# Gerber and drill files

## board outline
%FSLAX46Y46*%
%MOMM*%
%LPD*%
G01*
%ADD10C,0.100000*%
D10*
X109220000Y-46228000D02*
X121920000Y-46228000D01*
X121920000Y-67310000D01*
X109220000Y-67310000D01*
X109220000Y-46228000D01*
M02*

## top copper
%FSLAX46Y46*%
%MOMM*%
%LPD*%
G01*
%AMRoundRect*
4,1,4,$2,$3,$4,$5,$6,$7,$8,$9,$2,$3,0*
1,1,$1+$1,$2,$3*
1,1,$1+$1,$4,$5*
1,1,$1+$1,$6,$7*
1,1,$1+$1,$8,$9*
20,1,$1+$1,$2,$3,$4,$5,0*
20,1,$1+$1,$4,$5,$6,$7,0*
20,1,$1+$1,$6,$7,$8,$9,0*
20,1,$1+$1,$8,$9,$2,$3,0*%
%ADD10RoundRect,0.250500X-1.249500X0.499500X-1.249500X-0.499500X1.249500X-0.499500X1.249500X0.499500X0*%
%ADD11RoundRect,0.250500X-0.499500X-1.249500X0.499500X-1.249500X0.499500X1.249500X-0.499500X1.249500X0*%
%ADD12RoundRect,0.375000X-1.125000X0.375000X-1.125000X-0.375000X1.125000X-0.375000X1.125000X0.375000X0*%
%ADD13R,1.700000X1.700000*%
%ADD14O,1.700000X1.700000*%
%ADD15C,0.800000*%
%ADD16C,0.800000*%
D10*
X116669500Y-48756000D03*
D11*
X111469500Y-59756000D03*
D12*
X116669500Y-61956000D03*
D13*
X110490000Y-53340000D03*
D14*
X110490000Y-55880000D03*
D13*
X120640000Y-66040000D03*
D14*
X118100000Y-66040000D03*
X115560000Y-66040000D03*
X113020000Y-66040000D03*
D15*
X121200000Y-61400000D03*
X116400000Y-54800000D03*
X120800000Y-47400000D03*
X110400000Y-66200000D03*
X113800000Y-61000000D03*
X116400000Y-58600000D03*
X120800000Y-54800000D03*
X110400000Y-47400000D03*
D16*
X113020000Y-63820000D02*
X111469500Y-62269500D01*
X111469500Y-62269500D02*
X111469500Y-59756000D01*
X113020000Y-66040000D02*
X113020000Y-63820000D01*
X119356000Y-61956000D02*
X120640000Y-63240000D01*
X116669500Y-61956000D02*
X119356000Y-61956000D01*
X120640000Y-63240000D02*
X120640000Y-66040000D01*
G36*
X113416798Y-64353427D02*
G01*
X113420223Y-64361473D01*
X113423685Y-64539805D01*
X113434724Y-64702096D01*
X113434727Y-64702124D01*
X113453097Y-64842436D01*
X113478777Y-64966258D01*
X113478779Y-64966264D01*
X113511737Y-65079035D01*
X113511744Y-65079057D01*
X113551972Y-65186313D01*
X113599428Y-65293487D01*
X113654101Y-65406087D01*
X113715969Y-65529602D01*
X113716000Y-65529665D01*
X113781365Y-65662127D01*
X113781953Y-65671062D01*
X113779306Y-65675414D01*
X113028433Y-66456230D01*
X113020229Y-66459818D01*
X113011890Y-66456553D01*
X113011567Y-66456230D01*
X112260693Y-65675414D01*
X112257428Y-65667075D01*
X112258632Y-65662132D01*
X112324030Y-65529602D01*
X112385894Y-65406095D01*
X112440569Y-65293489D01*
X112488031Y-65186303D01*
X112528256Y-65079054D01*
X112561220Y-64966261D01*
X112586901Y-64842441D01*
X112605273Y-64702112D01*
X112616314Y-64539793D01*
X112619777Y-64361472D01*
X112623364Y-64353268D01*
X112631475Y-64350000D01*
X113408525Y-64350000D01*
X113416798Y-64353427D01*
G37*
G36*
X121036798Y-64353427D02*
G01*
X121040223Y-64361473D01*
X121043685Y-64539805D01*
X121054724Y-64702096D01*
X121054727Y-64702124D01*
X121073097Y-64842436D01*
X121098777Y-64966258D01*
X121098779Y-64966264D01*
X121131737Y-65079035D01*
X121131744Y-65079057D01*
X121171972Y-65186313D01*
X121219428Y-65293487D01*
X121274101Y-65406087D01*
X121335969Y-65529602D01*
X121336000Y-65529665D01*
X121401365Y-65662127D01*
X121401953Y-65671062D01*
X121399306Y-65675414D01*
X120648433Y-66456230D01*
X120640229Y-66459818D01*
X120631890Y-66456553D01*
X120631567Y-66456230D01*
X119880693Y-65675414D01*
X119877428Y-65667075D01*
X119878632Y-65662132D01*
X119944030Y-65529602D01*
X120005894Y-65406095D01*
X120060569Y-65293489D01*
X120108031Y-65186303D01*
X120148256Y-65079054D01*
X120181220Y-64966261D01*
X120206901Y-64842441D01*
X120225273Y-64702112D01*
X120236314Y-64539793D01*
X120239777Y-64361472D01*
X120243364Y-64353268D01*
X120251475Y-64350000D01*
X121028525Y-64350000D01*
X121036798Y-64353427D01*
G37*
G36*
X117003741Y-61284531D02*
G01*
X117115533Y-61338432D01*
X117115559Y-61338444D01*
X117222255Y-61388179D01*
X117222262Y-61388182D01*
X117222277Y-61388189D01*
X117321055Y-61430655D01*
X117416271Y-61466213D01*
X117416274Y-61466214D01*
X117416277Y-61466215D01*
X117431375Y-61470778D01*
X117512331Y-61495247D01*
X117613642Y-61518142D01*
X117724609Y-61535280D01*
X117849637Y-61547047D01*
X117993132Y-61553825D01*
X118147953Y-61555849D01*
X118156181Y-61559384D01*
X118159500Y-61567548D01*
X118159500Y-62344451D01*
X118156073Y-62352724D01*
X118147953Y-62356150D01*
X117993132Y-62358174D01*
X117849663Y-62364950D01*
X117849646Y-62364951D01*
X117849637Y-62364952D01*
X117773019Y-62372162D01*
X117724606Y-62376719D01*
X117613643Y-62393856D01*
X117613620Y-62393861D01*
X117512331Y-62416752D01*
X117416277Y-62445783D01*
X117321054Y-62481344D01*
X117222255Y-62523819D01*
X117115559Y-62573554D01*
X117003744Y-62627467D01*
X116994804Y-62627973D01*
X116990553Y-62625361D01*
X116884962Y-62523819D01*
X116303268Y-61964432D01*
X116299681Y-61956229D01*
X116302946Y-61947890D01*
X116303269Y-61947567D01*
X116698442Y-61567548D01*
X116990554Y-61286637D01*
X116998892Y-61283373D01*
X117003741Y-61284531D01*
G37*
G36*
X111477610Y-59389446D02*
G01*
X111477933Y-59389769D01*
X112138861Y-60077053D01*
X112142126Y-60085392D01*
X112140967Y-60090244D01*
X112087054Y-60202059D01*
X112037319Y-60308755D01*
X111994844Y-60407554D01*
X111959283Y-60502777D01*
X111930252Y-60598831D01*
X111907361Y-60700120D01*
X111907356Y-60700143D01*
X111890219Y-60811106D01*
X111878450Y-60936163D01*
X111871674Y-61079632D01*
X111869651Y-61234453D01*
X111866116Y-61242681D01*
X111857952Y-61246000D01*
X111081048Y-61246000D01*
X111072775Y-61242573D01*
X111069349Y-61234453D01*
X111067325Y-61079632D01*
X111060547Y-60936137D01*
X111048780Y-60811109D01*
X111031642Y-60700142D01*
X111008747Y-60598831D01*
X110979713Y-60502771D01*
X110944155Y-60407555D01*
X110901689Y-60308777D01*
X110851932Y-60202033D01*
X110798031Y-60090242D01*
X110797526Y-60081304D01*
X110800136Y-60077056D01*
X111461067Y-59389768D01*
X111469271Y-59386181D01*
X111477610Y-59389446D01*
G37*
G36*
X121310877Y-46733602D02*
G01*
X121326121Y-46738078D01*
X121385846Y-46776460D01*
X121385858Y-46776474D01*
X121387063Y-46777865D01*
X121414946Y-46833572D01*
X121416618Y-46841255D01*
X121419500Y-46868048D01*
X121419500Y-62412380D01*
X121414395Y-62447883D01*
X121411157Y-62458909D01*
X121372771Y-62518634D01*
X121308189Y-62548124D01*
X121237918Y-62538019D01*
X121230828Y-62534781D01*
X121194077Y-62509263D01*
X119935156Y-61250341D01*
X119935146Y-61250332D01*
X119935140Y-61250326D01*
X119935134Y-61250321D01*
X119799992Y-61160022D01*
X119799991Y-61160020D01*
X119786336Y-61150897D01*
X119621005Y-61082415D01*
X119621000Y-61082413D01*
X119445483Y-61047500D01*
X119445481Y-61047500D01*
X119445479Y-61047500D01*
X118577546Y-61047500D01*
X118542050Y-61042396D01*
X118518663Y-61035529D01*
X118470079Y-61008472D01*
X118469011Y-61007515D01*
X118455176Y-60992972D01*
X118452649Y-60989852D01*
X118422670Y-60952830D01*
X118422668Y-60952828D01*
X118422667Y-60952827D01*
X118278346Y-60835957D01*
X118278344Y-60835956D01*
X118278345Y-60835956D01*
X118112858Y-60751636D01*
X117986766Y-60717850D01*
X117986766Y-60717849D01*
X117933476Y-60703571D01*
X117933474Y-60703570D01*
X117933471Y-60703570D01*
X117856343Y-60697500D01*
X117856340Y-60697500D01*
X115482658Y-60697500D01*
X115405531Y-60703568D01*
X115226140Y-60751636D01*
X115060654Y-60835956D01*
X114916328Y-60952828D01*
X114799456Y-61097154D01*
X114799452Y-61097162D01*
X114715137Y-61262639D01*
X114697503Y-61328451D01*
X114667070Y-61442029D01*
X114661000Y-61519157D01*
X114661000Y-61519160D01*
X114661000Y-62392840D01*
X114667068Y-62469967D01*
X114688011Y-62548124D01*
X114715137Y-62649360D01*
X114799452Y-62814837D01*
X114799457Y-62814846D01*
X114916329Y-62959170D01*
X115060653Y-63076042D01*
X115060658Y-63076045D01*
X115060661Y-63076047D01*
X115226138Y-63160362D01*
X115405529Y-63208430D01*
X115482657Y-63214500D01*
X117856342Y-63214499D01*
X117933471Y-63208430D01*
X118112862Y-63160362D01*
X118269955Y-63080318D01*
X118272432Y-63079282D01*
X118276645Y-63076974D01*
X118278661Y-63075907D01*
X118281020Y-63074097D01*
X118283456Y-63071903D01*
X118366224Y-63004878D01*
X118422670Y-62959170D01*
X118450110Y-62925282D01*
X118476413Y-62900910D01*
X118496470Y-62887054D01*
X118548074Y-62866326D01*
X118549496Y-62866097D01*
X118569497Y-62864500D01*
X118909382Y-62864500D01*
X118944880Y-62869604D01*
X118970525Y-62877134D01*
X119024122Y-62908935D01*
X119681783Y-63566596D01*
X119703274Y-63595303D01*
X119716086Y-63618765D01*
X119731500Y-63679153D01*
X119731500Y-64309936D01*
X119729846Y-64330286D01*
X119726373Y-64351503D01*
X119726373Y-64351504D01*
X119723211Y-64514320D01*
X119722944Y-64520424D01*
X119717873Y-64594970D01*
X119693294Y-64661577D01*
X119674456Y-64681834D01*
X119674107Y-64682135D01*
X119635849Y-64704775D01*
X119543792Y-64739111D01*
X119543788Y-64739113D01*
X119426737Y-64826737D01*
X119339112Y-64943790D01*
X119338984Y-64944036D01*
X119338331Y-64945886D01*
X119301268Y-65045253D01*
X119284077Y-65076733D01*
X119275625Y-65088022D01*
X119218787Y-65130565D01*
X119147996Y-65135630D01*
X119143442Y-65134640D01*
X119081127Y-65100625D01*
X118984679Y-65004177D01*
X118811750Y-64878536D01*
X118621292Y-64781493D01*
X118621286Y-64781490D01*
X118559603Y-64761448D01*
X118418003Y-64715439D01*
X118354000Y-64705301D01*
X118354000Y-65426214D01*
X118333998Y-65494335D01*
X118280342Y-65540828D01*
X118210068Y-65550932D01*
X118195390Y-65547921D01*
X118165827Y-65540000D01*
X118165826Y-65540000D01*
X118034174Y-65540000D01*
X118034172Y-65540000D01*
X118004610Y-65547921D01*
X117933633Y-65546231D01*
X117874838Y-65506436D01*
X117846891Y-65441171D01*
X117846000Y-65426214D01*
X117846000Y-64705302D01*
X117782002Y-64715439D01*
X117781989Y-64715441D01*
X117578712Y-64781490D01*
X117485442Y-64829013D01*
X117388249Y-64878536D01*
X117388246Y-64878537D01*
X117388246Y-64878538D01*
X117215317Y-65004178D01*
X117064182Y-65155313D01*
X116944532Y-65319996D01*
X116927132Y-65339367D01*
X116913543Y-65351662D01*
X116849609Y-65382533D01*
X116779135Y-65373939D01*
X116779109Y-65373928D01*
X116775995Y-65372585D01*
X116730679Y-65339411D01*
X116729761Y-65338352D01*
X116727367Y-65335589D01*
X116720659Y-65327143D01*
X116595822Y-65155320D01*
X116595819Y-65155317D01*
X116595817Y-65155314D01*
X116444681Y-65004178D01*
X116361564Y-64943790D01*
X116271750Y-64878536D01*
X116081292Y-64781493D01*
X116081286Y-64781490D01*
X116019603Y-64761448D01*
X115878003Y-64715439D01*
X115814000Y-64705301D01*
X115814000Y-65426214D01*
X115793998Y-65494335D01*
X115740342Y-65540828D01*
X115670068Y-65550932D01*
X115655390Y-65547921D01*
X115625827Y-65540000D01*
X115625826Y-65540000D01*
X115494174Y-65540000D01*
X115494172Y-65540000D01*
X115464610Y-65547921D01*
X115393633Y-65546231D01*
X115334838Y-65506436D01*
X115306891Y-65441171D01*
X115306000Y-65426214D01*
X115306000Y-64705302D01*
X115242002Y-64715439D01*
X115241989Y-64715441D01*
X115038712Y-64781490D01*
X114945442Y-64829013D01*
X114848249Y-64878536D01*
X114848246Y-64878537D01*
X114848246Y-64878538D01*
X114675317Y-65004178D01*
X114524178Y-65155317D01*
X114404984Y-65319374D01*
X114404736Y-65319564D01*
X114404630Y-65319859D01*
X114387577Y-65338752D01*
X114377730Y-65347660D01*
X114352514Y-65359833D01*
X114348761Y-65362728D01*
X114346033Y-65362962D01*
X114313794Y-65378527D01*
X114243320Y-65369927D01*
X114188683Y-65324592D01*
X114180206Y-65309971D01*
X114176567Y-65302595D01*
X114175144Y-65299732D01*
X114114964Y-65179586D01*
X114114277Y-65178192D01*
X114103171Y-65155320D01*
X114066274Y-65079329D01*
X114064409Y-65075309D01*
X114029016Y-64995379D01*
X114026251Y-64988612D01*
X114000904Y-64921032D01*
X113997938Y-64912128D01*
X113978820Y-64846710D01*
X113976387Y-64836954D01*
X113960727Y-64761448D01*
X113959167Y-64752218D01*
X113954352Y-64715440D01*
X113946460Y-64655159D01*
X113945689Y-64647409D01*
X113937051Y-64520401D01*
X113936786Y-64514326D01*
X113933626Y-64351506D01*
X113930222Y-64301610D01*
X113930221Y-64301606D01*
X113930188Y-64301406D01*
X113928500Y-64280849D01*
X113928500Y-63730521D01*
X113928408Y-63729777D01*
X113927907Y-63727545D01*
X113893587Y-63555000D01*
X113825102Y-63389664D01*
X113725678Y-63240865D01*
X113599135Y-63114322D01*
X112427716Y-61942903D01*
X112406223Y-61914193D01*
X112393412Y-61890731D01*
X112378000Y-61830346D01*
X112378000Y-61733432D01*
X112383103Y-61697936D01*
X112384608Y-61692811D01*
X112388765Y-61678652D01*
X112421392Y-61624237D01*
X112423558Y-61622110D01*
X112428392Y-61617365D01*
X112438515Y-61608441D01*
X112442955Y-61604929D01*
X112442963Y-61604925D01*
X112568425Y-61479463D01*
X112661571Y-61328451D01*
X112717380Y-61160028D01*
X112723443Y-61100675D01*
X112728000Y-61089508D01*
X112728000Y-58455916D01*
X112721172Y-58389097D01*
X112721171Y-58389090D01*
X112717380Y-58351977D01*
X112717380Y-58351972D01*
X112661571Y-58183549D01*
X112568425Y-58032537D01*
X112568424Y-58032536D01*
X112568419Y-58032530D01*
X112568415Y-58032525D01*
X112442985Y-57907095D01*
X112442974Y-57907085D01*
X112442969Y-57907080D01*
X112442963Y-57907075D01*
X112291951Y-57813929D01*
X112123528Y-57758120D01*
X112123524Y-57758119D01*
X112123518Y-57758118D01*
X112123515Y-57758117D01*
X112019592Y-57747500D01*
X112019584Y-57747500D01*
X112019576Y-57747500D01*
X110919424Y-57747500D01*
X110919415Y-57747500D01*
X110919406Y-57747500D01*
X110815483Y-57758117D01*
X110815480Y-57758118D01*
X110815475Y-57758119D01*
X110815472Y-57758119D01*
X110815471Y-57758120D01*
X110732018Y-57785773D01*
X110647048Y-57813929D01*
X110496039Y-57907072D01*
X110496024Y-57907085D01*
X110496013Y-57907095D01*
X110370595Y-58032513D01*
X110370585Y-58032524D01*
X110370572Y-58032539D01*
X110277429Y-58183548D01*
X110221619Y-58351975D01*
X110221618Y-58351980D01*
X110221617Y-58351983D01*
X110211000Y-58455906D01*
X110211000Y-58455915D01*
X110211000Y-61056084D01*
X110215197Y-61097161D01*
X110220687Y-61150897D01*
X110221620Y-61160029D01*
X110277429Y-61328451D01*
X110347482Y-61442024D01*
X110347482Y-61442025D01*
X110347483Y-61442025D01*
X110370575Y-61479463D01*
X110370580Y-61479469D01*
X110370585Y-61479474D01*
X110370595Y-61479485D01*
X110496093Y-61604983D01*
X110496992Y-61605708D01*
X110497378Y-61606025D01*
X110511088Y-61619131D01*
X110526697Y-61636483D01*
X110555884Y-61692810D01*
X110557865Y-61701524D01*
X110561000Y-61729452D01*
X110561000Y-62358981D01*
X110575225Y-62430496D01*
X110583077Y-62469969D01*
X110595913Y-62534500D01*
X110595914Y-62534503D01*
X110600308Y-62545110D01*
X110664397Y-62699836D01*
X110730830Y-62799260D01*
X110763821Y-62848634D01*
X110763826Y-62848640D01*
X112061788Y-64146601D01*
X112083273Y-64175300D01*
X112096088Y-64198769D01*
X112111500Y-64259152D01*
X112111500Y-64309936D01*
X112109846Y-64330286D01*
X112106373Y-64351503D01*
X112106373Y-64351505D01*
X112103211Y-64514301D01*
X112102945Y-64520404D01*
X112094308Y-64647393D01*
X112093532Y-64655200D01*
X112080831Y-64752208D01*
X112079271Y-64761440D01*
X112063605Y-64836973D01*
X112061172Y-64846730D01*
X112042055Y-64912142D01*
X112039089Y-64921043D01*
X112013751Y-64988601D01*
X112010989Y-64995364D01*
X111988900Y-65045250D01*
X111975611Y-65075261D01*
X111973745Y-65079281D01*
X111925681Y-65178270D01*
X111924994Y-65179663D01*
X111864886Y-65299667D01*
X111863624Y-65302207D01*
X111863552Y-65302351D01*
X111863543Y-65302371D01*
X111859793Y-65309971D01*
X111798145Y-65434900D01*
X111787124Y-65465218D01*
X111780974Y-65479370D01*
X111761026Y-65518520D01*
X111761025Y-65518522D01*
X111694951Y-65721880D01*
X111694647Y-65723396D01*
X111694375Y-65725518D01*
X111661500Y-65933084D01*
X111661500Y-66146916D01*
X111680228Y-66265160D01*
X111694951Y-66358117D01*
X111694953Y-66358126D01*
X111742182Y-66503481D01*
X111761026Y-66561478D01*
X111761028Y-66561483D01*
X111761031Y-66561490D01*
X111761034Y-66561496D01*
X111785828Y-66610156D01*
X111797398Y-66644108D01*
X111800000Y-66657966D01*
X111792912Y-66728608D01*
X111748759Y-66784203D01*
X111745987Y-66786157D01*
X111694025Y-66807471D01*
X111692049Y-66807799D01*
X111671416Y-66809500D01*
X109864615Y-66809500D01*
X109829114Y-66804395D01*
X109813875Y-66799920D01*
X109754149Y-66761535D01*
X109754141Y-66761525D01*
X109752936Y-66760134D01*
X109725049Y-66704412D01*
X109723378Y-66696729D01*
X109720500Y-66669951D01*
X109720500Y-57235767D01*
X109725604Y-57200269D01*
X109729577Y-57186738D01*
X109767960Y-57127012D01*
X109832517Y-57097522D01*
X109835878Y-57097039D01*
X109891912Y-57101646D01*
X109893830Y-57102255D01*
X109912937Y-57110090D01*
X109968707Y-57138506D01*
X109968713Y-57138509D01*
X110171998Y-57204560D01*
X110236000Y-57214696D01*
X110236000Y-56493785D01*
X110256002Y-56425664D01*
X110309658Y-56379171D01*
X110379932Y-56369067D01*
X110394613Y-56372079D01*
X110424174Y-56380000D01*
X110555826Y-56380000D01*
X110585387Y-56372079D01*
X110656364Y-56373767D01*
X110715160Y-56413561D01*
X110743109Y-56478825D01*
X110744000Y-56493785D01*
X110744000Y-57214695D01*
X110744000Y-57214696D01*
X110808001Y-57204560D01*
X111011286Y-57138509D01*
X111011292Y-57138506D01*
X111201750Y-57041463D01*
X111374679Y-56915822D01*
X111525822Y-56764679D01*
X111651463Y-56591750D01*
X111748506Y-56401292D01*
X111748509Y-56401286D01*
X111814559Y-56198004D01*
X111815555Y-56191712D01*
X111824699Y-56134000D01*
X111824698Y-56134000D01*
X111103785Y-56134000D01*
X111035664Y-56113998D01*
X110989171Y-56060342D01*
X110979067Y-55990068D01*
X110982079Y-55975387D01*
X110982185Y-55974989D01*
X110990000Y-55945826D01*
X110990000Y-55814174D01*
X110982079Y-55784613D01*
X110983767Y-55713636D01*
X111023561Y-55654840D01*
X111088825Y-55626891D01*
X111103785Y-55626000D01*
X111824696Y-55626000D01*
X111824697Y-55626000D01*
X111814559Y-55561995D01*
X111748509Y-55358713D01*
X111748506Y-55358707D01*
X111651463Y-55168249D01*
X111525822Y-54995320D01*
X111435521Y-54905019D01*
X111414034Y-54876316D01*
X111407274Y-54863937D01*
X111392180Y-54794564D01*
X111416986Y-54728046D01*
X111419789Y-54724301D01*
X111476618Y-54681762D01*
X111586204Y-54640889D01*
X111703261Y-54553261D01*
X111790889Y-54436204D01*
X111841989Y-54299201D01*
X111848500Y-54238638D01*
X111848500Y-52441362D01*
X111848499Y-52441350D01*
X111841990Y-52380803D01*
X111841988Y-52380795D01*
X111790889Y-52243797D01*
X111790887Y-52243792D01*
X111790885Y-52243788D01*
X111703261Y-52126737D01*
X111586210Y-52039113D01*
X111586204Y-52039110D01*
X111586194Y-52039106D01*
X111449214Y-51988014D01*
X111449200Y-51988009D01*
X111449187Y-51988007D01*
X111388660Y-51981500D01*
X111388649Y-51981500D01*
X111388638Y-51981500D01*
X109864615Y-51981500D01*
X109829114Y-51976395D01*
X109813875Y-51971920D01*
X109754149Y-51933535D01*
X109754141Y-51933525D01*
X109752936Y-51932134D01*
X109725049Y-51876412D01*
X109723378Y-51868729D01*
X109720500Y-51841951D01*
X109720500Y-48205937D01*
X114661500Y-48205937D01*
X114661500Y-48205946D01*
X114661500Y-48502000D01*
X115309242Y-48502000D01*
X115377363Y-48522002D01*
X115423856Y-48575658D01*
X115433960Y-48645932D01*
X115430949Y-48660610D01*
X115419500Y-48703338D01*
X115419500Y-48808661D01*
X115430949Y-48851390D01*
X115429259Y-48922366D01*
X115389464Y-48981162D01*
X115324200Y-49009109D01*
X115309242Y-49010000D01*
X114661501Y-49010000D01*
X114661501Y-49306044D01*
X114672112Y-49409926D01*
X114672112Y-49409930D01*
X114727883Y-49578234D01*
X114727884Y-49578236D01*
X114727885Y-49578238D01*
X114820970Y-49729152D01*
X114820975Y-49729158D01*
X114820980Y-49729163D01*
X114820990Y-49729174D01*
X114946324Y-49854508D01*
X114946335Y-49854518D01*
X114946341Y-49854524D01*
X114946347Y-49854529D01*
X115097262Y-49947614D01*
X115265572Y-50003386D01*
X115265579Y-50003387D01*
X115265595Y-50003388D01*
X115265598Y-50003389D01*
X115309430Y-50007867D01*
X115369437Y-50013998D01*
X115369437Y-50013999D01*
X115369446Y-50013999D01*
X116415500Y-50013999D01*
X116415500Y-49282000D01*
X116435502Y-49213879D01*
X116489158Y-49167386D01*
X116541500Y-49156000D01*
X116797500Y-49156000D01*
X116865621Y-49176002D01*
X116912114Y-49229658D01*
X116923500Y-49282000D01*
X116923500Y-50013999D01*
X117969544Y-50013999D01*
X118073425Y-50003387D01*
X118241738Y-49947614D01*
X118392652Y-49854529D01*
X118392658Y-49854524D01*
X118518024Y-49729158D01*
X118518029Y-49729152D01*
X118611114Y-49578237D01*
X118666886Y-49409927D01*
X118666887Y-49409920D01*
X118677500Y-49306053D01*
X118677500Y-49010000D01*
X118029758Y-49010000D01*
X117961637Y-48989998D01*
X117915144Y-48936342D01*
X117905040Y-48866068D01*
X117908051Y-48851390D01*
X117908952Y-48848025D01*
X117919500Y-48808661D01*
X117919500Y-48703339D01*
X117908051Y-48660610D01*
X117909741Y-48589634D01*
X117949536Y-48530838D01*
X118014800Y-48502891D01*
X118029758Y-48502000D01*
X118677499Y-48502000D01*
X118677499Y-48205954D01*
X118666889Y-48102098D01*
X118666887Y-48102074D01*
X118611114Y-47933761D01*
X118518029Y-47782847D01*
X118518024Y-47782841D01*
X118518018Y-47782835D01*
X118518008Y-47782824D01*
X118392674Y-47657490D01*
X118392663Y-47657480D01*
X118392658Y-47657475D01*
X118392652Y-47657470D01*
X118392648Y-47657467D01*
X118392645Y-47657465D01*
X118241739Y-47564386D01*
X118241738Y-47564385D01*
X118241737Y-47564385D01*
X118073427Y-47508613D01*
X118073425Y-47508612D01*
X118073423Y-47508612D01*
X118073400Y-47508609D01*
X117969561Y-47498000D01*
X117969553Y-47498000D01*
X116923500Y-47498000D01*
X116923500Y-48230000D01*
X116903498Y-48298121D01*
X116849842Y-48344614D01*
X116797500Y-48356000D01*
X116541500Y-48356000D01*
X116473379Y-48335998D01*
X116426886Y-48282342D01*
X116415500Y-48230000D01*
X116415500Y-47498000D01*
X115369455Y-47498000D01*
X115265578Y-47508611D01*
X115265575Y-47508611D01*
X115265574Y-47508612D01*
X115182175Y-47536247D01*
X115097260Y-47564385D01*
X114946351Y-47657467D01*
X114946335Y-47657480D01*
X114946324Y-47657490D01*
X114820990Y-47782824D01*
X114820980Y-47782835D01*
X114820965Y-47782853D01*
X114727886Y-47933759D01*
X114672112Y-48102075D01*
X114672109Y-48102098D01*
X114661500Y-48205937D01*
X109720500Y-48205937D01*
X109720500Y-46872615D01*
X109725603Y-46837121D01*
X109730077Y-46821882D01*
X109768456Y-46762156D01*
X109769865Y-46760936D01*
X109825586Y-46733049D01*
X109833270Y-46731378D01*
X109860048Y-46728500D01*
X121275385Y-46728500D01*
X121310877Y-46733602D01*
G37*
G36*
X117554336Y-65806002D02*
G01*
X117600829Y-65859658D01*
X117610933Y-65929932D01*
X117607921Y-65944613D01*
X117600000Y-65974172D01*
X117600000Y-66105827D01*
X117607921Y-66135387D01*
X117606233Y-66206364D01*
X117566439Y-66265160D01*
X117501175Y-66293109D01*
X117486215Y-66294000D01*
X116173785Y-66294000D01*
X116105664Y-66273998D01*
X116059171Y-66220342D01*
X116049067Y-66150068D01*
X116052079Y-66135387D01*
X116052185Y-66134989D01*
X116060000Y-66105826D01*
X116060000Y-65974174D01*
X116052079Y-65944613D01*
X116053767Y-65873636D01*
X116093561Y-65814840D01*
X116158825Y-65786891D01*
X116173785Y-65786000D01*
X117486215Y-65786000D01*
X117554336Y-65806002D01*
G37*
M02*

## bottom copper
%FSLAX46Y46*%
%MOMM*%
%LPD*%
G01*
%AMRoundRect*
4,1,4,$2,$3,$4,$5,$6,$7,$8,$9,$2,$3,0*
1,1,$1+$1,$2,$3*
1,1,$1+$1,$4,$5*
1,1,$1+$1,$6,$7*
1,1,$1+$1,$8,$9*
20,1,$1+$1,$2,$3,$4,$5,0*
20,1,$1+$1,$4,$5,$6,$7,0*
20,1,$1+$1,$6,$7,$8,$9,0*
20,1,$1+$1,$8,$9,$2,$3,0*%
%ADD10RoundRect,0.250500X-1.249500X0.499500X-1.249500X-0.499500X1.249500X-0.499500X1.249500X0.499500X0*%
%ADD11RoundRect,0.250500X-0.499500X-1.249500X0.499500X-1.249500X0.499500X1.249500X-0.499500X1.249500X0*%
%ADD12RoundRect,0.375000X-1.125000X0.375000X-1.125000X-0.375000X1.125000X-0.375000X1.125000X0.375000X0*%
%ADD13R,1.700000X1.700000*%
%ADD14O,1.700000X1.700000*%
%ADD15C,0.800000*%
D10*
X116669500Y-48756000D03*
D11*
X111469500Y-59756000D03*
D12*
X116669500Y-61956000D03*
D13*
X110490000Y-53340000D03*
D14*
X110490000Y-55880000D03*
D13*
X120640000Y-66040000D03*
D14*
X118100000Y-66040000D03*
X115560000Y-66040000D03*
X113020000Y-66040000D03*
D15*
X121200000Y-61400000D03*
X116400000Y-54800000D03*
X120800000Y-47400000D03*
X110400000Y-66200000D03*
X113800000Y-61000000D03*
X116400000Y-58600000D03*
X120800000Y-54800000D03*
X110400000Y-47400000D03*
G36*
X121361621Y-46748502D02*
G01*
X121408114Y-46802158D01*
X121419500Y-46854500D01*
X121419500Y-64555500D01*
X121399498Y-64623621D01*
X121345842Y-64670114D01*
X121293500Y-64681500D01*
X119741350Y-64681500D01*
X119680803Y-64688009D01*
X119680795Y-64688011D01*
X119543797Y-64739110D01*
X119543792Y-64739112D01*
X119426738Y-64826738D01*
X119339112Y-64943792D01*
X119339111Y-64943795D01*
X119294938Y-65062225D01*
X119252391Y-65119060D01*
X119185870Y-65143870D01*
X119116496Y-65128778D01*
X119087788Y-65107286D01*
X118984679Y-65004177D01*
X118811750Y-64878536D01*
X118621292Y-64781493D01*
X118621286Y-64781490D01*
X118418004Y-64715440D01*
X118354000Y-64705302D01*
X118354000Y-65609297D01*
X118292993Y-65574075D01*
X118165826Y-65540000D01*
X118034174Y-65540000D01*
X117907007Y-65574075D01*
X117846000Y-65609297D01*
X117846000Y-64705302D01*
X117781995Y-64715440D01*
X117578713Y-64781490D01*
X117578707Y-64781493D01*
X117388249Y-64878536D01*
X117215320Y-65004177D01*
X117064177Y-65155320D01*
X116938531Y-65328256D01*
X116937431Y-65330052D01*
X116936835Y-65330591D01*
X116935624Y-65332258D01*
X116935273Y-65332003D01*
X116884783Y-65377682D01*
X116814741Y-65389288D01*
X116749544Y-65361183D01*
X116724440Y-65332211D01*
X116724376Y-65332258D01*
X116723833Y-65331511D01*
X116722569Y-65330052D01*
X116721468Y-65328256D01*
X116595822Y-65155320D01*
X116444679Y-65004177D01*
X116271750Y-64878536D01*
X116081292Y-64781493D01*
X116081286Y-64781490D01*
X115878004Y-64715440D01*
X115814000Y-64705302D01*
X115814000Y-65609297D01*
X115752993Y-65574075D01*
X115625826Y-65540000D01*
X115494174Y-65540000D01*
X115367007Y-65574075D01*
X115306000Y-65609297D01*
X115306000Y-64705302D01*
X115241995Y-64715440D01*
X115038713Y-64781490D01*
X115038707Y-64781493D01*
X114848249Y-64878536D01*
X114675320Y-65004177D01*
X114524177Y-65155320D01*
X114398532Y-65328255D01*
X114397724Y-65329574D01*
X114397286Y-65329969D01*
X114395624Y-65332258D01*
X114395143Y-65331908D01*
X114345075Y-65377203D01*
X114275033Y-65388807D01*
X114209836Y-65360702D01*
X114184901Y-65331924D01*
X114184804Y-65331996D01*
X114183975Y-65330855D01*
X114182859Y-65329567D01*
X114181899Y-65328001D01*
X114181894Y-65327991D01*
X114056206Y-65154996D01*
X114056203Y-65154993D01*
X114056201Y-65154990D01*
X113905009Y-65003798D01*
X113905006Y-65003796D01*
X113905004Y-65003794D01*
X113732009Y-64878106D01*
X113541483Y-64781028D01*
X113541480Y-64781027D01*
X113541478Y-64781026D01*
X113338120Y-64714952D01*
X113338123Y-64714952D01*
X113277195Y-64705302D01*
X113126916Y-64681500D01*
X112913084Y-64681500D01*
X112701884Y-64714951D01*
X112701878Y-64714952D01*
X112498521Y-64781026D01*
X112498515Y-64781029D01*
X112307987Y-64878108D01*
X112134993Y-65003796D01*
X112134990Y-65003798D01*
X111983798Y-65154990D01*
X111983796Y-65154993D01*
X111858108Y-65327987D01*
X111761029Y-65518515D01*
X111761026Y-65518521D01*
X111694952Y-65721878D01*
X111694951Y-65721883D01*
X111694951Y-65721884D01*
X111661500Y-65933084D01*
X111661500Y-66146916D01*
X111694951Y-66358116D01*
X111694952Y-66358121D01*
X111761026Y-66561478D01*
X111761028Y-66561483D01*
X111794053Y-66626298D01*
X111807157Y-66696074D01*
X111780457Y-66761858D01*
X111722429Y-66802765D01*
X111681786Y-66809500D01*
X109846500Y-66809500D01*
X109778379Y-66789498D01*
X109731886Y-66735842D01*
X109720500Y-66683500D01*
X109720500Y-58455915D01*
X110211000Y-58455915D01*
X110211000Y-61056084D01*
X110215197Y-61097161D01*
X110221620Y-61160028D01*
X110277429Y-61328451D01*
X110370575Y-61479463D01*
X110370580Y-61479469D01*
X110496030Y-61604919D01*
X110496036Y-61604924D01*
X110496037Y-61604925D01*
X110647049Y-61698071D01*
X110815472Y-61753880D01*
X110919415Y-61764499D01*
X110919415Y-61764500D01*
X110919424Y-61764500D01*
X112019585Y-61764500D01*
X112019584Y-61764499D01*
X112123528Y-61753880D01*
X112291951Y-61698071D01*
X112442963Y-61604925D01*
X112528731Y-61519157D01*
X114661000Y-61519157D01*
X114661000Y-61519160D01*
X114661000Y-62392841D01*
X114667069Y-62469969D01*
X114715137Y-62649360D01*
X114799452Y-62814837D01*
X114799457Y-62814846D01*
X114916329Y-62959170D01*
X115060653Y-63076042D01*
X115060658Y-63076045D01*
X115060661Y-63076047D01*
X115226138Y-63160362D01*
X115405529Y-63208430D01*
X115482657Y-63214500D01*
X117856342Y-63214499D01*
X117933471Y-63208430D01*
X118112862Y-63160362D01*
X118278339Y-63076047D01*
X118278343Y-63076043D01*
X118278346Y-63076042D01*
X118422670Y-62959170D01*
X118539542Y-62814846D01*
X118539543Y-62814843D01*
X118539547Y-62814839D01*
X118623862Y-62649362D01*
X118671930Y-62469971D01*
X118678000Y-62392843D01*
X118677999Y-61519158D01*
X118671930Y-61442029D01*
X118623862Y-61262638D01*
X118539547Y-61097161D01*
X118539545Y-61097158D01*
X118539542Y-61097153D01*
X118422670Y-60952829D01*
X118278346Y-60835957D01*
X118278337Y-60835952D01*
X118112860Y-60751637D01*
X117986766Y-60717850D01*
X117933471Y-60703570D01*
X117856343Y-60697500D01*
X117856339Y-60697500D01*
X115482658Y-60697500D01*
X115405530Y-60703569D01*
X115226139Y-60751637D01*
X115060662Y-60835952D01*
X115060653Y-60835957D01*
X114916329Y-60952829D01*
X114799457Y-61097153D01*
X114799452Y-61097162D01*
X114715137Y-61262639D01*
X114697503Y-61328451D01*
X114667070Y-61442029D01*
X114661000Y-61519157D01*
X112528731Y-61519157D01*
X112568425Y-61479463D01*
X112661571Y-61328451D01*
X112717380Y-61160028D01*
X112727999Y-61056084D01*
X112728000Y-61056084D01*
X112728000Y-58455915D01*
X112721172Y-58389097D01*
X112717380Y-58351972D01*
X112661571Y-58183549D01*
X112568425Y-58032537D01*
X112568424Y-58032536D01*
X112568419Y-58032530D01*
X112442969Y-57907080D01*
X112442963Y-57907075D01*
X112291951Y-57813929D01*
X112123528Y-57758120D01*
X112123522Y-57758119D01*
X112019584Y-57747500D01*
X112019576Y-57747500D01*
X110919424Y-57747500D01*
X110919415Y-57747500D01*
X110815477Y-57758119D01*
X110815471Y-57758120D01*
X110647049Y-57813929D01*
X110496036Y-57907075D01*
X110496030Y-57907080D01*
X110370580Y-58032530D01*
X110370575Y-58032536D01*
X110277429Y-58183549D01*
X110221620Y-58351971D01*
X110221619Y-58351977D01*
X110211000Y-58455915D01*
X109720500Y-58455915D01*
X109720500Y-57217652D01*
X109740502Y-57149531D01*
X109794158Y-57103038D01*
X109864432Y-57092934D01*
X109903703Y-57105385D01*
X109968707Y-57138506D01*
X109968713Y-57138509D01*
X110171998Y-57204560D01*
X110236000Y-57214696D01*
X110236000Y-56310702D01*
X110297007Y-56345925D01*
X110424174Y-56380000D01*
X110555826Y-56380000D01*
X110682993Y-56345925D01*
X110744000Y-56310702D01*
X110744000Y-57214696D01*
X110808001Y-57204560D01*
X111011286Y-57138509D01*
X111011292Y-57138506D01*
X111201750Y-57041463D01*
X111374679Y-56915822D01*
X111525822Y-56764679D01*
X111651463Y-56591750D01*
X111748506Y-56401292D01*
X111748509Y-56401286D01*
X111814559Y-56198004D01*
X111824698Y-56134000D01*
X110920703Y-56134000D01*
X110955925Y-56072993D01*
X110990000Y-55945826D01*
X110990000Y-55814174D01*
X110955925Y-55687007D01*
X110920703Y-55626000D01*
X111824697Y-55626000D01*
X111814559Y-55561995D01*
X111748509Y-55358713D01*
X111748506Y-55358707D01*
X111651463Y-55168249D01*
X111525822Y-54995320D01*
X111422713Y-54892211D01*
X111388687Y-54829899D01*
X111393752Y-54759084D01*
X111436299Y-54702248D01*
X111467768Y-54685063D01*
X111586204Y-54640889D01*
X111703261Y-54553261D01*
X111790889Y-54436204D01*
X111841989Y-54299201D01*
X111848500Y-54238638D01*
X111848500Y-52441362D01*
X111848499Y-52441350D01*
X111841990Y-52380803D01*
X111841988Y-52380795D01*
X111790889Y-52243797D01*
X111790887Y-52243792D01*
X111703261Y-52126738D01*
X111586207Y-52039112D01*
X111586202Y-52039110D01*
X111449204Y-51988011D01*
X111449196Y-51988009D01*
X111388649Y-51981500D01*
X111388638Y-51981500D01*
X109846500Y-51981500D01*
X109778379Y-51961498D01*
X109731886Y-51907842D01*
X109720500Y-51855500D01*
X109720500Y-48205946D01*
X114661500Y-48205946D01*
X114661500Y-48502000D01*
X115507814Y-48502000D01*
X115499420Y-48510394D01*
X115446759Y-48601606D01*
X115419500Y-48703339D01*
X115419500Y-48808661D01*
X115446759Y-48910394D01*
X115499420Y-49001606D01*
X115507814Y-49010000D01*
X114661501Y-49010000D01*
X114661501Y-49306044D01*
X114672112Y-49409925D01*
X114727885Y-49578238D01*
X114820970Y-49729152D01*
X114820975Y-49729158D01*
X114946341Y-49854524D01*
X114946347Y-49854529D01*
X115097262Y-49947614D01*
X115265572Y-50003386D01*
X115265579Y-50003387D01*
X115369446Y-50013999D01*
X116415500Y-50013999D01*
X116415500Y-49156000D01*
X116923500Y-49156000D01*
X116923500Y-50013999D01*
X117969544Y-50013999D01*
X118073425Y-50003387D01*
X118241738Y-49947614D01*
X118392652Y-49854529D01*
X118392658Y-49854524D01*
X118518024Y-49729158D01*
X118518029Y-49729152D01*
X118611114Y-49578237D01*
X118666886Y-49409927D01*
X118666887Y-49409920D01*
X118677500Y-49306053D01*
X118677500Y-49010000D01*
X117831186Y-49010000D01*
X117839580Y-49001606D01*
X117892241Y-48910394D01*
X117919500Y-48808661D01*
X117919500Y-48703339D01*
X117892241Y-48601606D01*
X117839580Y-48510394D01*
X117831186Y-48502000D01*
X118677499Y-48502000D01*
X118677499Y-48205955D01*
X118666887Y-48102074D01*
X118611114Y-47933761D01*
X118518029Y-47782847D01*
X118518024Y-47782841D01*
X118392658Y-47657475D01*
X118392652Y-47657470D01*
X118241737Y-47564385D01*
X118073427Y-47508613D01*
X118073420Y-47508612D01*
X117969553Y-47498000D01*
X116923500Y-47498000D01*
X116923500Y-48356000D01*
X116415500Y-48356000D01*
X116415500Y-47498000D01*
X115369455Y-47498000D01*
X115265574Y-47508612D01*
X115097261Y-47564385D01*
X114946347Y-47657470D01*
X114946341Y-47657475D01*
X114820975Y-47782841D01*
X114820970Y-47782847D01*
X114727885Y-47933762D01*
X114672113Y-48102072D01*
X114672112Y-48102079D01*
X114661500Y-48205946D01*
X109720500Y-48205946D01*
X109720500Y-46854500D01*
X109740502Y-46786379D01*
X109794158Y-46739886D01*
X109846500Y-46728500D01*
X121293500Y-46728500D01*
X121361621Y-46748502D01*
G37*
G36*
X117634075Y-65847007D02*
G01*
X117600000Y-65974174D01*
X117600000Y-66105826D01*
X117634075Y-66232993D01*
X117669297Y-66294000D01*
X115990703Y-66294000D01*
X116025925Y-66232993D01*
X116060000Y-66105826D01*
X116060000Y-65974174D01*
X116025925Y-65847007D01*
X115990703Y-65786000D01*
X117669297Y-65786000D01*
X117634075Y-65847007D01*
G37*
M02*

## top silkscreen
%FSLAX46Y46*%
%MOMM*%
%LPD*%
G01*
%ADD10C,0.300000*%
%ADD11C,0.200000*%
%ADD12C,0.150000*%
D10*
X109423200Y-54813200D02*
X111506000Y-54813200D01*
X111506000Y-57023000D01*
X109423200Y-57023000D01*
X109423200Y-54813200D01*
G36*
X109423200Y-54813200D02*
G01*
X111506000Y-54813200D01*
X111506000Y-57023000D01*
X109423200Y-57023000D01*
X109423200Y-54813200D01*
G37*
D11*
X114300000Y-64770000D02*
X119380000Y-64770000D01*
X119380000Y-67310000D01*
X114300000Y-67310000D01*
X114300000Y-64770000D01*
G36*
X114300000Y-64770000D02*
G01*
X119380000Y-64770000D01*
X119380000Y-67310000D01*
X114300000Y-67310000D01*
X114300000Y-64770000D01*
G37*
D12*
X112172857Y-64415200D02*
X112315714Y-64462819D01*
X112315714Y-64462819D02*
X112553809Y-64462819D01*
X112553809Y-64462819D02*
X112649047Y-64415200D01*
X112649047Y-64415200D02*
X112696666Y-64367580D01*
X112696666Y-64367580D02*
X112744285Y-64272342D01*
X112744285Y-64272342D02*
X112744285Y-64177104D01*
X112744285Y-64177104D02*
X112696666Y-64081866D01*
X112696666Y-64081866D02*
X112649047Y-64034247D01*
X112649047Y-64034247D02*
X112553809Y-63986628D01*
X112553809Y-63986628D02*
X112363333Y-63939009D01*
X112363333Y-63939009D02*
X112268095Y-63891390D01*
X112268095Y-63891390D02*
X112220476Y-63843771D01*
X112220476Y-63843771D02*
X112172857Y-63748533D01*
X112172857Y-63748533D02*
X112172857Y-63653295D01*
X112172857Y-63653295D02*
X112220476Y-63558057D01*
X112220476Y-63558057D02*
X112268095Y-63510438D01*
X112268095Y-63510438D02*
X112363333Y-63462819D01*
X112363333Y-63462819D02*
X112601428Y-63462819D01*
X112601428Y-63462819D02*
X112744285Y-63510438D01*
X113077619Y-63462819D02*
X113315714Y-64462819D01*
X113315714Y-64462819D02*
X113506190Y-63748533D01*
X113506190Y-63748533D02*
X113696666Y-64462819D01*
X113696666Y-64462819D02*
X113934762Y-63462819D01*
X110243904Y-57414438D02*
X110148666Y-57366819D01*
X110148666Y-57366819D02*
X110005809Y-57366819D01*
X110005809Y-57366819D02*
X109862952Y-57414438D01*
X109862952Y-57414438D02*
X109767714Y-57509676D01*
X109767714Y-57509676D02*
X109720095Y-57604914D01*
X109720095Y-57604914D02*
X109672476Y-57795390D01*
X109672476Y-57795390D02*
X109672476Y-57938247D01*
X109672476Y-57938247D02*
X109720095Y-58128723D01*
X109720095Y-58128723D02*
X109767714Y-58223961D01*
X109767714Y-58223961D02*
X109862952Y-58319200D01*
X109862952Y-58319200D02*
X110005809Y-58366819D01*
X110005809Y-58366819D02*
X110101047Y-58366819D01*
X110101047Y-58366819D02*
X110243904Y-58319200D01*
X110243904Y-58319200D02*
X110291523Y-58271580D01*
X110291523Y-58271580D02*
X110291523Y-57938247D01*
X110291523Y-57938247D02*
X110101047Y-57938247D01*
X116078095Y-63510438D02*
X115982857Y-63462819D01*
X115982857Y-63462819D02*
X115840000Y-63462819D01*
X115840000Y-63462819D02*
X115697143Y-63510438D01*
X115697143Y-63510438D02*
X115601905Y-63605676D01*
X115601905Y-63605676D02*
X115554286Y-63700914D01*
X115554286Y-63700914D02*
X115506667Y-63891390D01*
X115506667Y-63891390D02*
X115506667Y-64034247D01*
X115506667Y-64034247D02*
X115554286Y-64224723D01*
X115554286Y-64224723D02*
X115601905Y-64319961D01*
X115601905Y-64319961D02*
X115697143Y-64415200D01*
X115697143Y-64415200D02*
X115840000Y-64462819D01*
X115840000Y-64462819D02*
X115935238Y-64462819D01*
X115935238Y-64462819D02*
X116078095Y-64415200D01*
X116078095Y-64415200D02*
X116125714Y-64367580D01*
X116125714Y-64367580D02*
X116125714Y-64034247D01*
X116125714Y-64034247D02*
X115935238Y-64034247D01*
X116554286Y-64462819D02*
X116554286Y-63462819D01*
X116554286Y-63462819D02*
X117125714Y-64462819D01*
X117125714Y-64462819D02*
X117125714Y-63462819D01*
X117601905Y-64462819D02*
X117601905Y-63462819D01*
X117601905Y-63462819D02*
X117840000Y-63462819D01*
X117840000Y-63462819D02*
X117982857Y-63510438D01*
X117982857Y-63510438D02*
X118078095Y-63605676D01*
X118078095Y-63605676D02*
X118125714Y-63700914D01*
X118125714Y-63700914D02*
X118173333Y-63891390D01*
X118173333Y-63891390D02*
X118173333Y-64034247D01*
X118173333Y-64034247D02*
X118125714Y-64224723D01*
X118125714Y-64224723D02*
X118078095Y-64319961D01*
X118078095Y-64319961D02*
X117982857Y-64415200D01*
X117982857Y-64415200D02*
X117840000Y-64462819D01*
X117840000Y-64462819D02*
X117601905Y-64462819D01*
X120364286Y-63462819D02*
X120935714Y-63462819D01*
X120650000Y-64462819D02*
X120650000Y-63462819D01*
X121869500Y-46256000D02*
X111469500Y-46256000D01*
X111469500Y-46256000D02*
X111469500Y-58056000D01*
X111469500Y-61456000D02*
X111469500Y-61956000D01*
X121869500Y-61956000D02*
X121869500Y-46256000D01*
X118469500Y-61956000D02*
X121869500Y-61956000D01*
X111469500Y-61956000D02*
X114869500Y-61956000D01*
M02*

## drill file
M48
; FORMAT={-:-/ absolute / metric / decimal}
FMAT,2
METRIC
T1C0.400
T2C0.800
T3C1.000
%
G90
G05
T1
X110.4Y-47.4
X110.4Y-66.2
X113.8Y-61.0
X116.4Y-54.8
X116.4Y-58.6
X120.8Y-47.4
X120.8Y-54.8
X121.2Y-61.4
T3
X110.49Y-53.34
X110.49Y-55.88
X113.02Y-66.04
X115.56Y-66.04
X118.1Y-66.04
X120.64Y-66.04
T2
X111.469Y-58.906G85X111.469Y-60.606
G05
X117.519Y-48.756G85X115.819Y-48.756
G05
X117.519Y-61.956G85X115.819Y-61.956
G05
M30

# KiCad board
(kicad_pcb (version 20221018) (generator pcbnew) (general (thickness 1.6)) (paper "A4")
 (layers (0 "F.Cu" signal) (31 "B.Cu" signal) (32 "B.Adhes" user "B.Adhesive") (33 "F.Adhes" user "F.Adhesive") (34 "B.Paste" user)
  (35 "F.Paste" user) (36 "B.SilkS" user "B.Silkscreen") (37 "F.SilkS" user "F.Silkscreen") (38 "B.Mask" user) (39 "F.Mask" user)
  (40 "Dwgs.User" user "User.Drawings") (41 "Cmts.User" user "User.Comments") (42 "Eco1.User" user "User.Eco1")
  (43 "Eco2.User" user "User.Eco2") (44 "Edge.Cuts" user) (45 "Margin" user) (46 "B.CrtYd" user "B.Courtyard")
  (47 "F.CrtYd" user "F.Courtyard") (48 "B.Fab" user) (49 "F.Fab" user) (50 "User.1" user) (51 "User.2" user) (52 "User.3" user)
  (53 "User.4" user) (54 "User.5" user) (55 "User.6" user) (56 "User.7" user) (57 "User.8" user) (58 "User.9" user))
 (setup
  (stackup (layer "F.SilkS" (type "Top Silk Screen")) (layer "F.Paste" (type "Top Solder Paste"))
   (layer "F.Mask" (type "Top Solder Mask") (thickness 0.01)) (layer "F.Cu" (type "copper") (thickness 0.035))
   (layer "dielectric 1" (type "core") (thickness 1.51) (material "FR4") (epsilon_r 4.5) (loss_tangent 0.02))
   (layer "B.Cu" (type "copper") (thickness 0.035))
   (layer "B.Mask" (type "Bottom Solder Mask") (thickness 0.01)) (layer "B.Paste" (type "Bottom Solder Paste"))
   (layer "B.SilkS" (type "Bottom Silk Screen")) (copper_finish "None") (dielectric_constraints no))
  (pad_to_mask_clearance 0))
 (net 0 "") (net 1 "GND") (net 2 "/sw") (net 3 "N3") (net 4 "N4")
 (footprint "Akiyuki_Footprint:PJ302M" (layer "F.Cu") (at 116.6695 46.256 -90)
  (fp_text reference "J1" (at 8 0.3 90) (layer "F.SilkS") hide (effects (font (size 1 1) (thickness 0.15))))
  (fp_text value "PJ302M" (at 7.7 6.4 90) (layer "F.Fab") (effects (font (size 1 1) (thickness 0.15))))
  (fp_line (start 0 -5.2) (end 0 5.2) (stroke (width 0.15) (type solid)) (layer "F.SilkS"))
  (fp_line (start 0 5.2) (end 11.8 5.2) (stroke (width 0.15) (type solid)) (layer "F.SilkS"))
  (fp_line (start 15.2 5.2) (end 15.7 5.2) (stroke (width 0.15) (type solid)) (layer "F.SilkS"))
  (fp_line (start 15.7 -5.2) (end 0 -5.2) (stroke (width 0.15) (type solid)) (layer "F.SilkS"))
  (fp_line (start 15.7 -1.8) (end 15.7 -5.2) (stroke (width 0.15) (type solid)) (layer "F.SilkS"))
  (fp_line (start 15.7 5.2) (end 15.7 1.8) (stroke (width 0.15) (type solid)) (layer "F.SilkS"))
  (pad "1" thru_hole roundrect (at 2.5 0 270) (size 1.5 3) (drill oval 0.8 2.5) (layers "*.Cu" "*.Mask") (roundrect_rratio 0.167)
   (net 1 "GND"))
  (pad "2" thru_hole roundrect (at 13.5 5.2) (size 1.5 3) (drill oval 0.8 2.5) (layers "*.Cu" "*.Mask") (roundrect_rratio 0.167)
   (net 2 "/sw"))
  (pad "3" thru_hole roundrect (at 15.7 0 270) (size 1.5 3) (drill oval 0.8 2.5) (layers "*.Cu" "*.Mask") (roundrect_rratio 0.25)
   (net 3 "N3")))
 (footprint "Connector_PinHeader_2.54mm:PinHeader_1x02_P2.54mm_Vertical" (layer "B.Cu") (at 110.49 53.34 180)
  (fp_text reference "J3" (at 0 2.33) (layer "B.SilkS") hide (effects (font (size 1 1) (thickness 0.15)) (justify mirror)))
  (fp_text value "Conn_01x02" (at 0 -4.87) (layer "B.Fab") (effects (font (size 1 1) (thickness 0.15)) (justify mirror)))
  (pad "1" thru_hole rect (at 0 0 180) (size 1.7 1.7) (drill 1) (layers "*.Cu" "*.Mask") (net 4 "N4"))
  (pad "2" thru_hole oval (at 0 -2.54 180) (size 1.7 1.7) (drill 1) (layers "*.Cu" "*.Mask") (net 1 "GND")))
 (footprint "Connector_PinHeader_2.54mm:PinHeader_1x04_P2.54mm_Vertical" (layer "B.Cu") (at 120.64 66.04 90)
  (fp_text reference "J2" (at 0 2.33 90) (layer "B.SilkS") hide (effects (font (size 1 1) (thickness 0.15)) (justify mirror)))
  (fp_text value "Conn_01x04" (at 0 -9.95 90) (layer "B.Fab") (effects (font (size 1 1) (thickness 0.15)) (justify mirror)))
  (pad "1" thru_hole rect (at 0 0 90) (size 1.7 1.7) (drill 1) (layers "*.Cu" "*.Mask") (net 3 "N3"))
  (pad "2" thru_hole oval (at 0 -2.54 90) (size 1.7 1.7) (drill 1) (layers "*.Cu" "*.Mask") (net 1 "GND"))
  (pad "3" thru_hole oval (at 0 -5.08 90) (size 1.7 1.7) (drill 1) (layers "*.Cu" "*.Mask") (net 1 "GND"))
  (pad "4" thru_hole oval (at 0 -7.62 90) (size 1.7 1.7) (drill 1) (layers "*.Cu" "*.Mask") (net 2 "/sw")))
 (gr_rect (start 109.4232 54.8132) (end 111.506 57.023) (stroke (width 0.3) (type solid)) (fill solid) (layer "F.SilkS"))
 (gr_rect (start 114.3 64.77) (end 119.38 67.31) (stroke (width 0.2) (type solid)) (fill solid) (layer "F.SilkS"))
 (gr_rect (start 109.22 46.228) (end 121.92 67.31) (stroke (width 0.1) (type solid)) (fill none) (layer "Edge.Cuts"))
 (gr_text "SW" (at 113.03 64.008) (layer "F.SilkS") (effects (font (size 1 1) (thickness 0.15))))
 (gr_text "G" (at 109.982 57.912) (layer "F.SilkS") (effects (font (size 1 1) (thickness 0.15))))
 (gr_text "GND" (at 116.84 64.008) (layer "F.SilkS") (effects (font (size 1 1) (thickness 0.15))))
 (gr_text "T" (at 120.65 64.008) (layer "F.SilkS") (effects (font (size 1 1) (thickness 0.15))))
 (via (at 121.2 61.4) (size 0.8) (drill 0.4) (layers "F.Cu" "B.Cu") (free) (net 1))
 (via (at 116.4 54.8) (size 0.8) (drill 0.4) (layers "F.Cu" "B.Cu") (free) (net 1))
 (via (at 120.8 47.4) (size 0.8) (drill 0.4) (layers "F.Cu" "B.Cu") (free) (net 1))
 (via (at 110.4 66.2) (size 0.8) (drill 0.4) (layers "F.Cu" "B.Cu") (free) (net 1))
 (via (at 113.8 61) (size 0.8) (drill 0.4) (layers "F.Cu" "B.Cu") (free) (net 1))
 (via (at 116.4 58.6) (size 0.8) (drill 0.4) (layers "F.Cu" "B.Cu") (free) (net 1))
 (via (at 120.8 54.8) (size 0.8) (drill 0.4) (layers "F.Cu" "B.Cu") (free) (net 1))
 (via (at 110.4 47.4) (size 0.8) (drill 0.4) (layers "F.Cu" "B.Cu") (free) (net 1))
 (segment (start 113.02 63.82) (end 111.4695 62.2695) (width 0.8) (layer "F.Cu") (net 2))
 (segment (start 111.4695 62.2695) (end 111.4695 59.756) (width 0.8) (layer "F.Cu") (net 2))
 (segment (start 113.02 66.04) (end 113.02 63.82) (width 0.8) (layer "F.Cu") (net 2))
 (segment (start 119.356 61.956) (end 120.64 63.24) (width 0.8) (layer "F.Cu") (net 3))
 (segment (start 116.6695 61.956) (end 119.356 61.956) (width 0.8) (layer "F.Cu") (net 3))
 (segment (start 120.64 63.24) (end 120.64 66.04) (width 0.8) (layer "F.Cu") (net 3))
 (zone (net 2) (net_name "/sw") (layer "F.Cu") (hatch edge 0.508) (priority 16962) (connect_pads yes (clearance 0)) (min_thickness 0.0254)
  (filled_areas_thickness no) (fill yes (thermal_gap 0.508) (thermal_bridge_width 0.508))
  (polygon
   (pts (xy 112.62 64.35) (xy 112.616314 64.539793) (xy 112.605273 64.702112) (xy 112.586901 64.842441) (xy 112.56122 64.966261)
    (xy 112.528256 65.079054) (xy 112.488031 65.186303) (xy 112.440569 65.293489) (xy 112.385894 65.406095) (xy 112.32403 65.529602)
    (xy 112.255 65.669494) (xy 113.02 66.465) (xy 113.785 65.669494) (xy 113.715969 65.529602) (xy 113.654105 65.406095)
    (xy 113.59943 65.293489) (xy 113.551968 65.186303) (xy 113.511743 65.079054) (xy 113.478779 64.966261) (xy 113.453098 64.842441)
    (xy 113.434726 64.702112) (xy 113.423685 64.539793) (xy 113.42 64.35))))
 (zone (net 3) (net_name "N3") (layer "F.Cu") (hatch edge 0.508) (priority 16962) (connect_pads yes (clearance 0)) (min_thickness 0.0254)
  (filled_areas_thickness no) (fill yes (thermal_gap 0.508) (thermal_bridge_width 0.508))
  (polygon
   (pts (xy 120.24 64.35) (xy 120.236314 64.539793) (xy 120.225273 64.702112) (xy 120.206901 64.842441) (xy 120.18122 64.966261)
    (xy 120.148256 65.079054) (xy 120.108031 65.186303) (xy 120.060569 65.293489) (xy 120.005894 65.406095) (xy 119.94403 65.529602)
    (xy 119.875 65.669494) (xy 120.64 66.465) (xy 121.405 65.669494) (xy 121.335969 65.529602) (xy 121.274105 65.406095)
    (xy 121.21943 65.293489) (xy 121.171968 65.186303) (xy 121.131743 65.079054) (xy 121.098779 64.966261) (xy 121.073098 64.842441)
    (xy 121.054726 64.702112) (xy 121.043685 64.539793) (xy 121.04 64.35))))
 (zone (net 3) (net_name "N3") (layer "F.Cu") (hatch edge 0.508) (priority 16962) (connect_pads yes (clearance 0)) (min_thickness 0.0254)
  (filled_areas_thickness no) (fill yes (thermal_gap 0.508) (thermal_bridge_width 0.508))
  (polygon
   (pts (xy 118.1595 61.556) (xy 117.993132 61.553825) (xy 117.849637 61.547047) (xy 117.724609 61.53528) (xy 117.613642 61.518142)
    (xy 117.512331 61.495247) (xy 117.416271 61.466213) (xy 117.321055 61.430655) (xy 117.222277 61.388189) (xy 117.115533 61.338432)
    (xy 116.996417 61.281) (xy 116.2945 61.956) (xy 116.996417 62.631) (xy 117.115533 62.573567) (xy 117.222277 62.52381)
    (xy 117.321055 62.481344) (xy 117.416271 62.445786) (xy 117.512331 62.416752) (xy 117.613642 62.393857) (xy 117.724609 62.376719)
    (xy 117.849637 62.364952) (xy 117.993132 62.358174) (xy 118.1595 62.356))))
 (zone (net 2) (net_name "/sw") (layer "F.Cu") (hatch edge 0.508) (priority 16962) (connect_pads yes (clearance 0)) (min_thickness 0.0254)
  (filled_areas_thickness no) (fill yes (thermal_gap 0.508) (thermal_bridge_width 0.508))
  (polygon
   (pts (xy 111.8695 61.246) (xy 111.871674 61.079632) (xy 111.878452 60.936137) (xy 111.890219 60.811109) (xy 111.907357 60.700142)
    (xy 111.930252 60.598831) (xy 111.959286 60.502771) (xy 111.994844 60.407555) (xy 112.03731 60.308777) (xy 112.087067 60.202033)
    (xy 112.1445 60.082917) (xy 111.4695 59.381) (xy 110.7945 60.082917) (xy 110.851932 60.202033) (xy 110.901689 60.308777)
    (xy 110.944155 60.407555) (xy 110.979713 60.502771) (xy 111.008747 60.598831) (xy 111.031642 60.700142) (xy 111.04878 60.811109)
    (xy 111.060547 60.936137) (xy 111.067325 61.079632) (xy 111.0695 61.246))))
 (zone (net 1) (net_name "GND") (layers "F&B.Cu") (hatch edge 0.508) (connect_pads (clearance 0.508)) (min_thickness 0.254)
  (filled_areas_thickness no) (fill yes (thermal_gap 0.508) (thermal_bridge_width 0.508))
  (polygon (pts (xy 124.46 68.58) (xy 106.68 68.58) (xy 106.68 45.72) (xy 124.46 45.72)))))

